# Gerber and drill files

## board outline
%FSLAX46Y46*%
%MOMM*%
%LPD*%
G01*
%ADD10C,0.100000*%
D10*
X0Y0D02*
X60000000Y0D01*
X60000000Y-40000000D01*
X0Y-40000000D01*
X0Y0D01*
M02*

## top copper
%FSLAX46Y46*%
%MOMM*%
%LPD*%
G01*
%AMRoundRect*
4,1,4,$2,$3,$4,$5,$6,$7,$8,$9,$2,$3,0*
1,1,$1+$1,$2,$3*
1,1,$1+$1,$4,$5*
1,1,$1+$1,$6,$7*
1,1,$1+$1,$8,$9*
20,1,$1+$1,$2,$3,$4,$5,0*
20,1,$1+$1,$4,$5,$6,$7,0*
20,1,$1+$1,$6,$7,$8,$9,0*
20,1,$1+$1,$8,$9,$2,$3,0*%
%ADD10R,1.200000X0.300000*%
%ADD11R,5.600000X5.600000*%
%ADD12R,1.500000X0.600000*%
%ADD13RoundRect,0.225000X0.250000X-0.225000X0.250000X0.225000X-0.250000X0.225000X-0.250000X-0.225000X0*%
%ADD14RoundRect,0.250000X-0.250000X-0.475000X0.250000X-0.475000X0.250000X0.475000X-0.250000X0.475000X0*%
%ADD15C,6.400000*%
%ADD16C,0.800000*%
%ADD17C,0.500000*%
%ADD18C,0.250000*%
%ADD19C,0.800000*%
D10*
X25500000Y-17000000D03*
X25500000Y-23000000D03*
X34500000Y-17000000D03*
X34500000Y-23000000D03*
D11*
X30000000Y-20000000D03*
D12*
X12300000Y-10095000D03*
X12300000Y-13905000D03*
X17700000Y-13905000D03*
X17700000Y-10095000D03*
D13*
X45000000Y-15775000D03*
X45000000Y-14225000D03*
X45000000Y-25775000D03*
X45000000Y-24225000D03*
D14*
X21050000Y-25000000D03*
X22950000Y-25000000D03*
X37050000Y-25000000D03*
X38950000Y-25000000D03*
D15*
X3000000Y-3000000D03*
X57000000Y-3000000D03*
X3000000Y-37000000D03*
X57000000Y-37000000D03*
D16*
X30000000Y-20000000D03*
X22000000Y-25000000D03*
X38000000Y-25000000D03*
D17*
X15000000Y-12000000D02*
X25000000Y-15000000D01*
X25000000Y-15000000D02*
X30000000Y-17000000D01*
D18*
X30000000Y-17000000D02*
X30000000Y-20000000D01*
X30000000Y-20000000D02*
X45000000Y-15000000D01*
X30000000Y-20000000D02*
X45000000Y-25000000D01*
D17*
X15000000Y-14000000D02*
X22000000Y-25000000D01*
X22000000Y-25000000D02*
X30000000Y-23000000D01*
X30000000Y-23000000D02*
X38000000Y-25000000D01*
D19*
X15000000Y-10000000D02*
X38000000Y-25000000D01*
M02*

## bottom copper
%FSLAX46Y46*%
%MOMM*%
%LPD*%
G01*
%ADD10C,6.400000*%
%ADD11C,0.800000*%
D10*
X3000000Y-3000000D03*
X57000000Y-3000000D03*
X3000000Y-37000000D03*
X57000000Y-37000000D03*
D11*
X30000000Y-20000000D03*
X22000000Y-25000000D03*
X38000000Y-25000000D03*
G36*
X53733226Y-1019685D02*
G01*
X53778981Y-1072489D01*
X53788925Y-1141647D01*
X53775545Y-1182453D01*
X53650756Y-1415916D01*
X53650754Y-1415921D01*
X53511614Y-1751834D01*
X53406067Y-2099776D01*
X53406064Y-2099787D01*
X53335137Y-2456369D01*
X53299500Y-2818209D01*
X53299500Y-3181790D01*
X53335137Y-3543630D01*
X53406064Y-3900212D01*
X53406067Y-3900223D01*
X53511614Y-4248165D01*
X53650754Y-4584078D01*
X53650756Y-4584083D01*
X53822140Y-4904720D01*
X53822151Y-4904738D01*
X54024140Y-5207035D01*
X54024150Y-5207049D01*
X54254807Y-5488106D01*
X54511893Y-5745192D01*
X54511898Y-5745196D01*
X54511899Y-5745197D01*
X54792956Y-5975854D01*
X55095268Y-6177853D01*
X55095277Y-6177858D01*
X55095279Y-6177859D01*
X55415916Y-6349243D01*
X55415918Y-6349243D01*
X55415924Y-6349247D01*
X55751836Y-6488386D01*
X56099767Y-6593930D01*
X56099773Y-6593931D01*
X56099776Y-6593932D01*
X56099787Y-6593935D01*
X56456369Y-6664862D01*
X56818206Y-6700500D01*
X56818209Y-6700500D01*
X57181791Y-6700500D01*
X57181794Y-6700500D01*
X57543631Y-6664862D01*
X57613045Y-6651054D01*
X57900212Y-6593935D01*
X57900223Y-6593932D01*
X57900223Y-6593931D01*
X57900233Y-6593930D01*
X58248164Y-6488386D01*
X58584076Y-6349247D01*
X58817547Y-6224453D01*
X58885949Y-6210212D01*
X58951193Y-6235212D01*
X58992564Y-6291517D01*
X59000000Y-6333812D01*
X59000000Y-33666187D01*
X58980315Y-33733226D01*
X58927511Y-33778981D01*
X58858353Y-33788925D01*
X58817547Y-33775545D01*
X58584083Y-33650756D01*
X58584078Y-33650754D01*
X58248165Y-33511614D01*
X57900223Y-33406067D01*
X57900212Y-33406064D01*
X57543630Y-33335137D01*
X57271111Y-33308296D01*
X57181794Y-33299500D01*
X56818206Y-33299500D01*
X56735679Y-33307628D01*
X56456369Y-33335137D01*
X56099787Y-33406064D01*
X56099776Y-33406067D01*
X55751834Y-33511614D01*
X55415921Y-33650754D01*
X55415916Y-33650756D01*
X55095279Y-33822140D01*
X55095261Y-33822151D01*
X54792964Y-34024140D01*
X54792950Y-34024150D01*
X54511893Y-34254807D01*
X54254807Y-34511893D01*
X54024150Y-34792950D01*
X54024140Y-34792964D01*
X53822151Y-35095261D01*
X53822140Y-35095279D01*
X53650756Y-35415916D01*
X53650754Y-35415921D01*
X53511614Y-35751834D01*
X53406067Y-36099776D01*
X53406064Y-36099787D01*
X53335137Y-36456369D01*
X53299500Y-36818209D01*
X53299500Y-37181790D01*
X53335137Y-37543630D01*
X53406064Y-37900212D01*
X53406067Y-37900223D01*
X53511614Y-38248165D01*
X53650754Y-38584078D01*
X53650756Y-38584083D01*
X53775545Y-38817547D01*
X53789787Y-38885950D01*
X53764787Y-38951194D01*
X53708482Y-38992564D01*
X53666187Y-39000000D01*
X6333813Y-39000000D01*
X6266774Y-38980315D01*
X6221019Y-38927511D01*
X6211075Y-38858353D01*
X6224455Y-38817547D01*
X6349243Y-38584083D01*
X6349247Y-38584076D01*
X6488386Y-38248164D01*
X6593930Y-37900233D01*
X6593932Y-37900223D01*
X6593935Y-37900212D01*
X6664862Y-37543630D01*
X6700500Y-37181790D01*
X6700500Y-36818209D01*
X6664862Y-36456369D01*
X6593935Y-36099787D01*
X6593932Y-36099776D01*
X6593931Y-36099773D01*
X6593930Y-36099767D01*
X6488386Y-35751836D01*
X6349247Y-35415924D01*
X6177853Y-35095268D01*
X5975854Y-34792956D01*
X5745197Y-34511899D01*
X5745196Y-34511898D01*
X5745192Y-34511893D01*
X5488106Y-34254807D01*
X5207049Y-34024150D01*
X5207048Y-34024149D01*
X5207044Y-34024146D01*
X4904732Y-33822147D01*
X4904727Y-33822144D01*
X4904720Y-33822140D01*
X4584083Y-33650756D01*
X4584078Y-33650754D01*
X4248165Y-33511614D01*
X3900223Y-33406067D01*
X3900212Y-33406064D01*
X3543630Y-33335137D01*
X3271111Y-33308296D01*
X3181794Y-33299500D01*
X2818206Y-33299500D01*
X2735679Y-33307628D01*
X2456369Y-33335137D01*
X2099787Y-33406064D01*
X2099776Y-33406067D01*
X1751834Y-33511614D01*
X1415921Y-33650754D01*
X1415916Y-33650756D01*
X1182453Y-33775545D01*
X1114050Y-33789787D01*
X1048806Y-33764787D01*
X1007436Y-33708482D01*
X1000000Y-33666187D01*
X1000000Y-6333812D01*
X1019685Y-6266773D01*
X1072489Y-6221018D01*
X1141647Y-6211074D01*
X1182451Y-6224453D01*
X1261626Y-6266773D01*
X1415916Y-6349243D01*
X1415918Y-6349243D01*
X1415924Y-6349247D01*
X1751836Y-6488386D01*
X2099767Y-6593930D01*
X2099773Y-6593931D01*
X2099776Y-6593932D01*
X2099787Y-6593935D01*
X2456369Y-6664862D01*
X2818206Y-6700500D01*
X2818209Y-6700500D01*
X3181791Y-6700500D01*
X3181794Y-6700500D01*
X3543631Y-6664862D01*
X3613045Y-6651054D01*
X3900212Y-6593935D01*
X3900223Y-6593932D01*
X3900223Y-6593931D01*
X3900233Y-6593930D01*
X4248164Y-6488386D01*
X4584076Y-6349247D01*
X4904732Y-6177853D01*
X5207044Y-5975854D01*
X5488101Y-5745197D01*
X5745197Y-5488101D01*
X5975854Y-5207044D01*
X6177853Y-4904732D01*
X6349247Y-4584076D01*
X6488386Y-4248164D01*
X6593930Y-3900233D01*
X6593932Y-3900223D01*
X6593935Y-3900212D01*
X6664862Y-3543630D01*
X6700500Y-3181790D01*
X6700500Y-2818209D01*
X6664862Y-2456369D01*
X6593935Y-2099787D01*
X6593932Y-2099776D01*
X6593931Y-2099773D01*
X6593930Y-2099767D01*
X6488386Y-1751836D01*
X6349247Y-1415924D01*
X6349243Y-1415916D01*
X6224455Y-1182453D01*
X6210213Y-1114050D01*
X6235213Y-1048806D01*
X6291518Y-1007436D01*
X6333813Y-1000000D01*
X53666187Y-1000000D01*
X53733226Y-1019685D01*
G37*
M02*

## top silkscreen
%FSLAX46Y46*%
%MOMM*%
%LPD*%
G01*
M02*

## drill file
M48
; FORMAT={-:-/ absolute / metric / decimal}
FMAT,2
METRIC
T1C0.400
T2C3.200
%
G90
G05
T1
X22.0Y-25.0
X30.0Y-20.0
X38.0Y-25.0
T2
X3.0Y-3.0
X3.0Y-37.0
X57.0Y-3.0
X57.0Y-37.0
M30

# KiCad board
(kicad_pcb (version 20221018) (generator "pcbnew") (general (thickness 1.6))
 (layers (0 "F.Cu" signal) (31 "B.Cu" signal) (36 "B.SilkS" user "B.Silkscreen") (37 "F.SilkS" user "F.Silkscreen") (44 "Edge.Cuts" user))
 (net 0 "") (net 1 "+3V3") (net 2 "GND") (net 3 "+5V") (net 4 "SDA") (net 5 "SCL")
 (gr_rect (start 0 0) (end 60 40) (layer "Edge.Cuts") (width 0.1))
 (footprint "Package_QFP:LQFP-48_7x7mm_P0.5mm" (at 30 20 0) (layer "F.Cu") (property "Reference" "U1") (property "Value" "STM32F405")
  (pad "1" smd rect (at -4.5 -3 0) (size 1.2 0.3) (layers "F.Cu") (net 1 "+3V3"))
  (pad "12" smd rect (at -4.5 3 0) (size 1.2 0.3) (layers "F.Cu") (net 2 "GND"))
  (pad "24" smd rect (at 4.5 -3 0) (size 1.2 0.3) (layers "F.Cu") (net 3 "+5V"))
  (pad "36" smd rect (at 4.5 3 0) (size 1.2 0.3) (layers "F.Cu") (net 2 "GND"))
  (pad "49" smd rect (at 0 0 0) (size 5.6 5.6) (layers "F.Cu") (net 2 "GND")))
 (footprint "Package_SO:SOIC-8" (at 15 12 0) (layer "F.Cu") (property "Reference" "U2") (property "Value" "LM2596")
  (pad "1" smd rect (at -2.7 -1.905 0) (size 1.5 0.6) (layers "F.Cu") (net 3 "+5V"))
  (pad "4" smd rect (at -2.7 1.905 0) (size 1.5 0.6) (layers "F.Cu") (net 2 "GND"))
  (pad "5" smd rect (at 2.7 1.905 0) (size 1.5 0.6) (layers "F.Cu") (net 1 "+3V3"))
  (pad "8" smd rect (at 2.7 -1.905 0) (size 1.5 0.6) (layers "F.Cu") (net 3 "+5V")))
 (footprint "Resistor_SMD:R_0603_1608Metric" (at 45 15 90) (layer "F.Cu") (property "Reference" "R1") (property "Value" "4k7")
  (pad "1" smd roundrect (at -0.775 0 90) (size 0.9 0.95) (layers "F.Cu") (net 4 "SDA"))
  (pad "2" smd roundrect (at 0.775 0 90) (size 0.9 0.95) (layers "F.Cu") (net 1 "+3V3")))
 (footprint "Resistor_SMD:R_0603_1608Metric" (at 45 25 90) (layer "F.Cu") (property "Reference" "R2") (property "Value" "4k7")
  (pad "1" smd roundrect (at -0.775 0 90) (size 0.9 0.95) (layers "F.Cu") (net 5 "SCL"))
  (pad "2" smd roundrect (at 0.775 0 90) (size 0.9 0.95) (layers "F.Cu") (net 1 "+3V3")))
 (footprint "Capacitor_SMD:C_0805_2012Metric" (at 22 25 0) (layer "F.Cu") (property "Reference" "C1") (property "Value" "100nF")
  (pad "1" smd roundrect (at -0.95 0 0) (size 1 1.45) (layers "F.Cu") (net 1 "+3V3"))
  (pad "2" smd roundrect (at 0.95 0 0) (size 1 1.45) (layers "F.Cu") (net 2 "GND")))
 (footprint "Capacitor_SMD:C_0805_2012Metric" (at 38 25 0) (layer "F.Cu") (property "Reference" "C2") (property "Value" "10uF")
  (pad "1" smd roundrect (at -0.95 0 0) (size 1 1.45) (layers "F.Cu") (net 3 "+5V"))
  (pad "2" smd roundrect (at 0.95 0 0) (size 1 1.45) (layers "F.Cu") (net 2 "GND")))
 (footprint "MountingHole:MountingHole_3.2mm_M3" (at 3 3 0) (layer "F.Cu") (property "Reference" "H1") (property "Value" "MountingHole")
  (pad "1" thru_hole circle (at 0 0) (size 6.4 6.4) (drill 3.2) (layers "*.Cu")))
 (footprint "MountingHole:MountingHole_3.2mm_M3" (at 57 3 0) (layer "F.Cu") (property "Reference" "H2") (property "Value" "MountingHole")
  (pad "1" thru_hole circle (at 0 0) (size 6.4 6.4) (drill 3.2) (layers "*.Cu")))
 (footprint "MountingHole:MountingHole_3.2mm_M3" (at 3 37 0) (layer "F.Cu") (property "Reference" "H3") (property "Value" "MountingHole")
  (pad "1" thru_hole circle (at 0 0) (size 6.4 6.4) (drill 3.2) (layers "*.Cu")))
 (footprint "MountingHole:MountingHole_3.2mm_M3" (at 57 37 0) (layer "F.Cu") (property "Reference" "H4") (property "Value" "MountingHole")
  (pad "1" thru_hole circle (at 0 0) (size 6.4 6.4) (drill 3.2) (layers "*.Cu")))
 (segment (start 15 12) (end 25 15) (width 0.5) (layer "F.Cu") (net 3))
 (segment (start 25 15) (end 30 17) (width 0.5) (layer "F.Cu") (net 3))
 (segment (start 30 17) (end 30 20) (width 0.25) (layer "F.Cu") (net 1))
 (segment (start 30 20) (end 45 15) (width 0.25) (layer "F.Cu") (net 4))
 (segment (start 30 20) (end 45 25) (width 0.25) (layer "F.Cu") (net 5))
 (segment (start 15 14) (end 22 25) (width 0.5) (layer "F.Cu") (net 2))
 (segment (start 22 25) (end 30 23) (width 0.5) (layer "F.Cu") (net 2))
 (segment (start 30 23) (end 38 25) (width 0.5) (layer "F.Cu") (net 2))
 (segment (start 15 10) (end 38 25) (width 0.8) (layer "F.Cu") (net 3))
 (via (at 30 20) (size 0.8) (drill 0.4) (layers "F.Cu" "B.Cu") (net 2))
 (via (at 22 25) (size 0.8) (drill 0.4) (layers "F.Cu" "B.Cu") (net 2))
 (via (at 38 25) (size 0.8) (drill 0.4) (layers "F.Cu" "B.Cu") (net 2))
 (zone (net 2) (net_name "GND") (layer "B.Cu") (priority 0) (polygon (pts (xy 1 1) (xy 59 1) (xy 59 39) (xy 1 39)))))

